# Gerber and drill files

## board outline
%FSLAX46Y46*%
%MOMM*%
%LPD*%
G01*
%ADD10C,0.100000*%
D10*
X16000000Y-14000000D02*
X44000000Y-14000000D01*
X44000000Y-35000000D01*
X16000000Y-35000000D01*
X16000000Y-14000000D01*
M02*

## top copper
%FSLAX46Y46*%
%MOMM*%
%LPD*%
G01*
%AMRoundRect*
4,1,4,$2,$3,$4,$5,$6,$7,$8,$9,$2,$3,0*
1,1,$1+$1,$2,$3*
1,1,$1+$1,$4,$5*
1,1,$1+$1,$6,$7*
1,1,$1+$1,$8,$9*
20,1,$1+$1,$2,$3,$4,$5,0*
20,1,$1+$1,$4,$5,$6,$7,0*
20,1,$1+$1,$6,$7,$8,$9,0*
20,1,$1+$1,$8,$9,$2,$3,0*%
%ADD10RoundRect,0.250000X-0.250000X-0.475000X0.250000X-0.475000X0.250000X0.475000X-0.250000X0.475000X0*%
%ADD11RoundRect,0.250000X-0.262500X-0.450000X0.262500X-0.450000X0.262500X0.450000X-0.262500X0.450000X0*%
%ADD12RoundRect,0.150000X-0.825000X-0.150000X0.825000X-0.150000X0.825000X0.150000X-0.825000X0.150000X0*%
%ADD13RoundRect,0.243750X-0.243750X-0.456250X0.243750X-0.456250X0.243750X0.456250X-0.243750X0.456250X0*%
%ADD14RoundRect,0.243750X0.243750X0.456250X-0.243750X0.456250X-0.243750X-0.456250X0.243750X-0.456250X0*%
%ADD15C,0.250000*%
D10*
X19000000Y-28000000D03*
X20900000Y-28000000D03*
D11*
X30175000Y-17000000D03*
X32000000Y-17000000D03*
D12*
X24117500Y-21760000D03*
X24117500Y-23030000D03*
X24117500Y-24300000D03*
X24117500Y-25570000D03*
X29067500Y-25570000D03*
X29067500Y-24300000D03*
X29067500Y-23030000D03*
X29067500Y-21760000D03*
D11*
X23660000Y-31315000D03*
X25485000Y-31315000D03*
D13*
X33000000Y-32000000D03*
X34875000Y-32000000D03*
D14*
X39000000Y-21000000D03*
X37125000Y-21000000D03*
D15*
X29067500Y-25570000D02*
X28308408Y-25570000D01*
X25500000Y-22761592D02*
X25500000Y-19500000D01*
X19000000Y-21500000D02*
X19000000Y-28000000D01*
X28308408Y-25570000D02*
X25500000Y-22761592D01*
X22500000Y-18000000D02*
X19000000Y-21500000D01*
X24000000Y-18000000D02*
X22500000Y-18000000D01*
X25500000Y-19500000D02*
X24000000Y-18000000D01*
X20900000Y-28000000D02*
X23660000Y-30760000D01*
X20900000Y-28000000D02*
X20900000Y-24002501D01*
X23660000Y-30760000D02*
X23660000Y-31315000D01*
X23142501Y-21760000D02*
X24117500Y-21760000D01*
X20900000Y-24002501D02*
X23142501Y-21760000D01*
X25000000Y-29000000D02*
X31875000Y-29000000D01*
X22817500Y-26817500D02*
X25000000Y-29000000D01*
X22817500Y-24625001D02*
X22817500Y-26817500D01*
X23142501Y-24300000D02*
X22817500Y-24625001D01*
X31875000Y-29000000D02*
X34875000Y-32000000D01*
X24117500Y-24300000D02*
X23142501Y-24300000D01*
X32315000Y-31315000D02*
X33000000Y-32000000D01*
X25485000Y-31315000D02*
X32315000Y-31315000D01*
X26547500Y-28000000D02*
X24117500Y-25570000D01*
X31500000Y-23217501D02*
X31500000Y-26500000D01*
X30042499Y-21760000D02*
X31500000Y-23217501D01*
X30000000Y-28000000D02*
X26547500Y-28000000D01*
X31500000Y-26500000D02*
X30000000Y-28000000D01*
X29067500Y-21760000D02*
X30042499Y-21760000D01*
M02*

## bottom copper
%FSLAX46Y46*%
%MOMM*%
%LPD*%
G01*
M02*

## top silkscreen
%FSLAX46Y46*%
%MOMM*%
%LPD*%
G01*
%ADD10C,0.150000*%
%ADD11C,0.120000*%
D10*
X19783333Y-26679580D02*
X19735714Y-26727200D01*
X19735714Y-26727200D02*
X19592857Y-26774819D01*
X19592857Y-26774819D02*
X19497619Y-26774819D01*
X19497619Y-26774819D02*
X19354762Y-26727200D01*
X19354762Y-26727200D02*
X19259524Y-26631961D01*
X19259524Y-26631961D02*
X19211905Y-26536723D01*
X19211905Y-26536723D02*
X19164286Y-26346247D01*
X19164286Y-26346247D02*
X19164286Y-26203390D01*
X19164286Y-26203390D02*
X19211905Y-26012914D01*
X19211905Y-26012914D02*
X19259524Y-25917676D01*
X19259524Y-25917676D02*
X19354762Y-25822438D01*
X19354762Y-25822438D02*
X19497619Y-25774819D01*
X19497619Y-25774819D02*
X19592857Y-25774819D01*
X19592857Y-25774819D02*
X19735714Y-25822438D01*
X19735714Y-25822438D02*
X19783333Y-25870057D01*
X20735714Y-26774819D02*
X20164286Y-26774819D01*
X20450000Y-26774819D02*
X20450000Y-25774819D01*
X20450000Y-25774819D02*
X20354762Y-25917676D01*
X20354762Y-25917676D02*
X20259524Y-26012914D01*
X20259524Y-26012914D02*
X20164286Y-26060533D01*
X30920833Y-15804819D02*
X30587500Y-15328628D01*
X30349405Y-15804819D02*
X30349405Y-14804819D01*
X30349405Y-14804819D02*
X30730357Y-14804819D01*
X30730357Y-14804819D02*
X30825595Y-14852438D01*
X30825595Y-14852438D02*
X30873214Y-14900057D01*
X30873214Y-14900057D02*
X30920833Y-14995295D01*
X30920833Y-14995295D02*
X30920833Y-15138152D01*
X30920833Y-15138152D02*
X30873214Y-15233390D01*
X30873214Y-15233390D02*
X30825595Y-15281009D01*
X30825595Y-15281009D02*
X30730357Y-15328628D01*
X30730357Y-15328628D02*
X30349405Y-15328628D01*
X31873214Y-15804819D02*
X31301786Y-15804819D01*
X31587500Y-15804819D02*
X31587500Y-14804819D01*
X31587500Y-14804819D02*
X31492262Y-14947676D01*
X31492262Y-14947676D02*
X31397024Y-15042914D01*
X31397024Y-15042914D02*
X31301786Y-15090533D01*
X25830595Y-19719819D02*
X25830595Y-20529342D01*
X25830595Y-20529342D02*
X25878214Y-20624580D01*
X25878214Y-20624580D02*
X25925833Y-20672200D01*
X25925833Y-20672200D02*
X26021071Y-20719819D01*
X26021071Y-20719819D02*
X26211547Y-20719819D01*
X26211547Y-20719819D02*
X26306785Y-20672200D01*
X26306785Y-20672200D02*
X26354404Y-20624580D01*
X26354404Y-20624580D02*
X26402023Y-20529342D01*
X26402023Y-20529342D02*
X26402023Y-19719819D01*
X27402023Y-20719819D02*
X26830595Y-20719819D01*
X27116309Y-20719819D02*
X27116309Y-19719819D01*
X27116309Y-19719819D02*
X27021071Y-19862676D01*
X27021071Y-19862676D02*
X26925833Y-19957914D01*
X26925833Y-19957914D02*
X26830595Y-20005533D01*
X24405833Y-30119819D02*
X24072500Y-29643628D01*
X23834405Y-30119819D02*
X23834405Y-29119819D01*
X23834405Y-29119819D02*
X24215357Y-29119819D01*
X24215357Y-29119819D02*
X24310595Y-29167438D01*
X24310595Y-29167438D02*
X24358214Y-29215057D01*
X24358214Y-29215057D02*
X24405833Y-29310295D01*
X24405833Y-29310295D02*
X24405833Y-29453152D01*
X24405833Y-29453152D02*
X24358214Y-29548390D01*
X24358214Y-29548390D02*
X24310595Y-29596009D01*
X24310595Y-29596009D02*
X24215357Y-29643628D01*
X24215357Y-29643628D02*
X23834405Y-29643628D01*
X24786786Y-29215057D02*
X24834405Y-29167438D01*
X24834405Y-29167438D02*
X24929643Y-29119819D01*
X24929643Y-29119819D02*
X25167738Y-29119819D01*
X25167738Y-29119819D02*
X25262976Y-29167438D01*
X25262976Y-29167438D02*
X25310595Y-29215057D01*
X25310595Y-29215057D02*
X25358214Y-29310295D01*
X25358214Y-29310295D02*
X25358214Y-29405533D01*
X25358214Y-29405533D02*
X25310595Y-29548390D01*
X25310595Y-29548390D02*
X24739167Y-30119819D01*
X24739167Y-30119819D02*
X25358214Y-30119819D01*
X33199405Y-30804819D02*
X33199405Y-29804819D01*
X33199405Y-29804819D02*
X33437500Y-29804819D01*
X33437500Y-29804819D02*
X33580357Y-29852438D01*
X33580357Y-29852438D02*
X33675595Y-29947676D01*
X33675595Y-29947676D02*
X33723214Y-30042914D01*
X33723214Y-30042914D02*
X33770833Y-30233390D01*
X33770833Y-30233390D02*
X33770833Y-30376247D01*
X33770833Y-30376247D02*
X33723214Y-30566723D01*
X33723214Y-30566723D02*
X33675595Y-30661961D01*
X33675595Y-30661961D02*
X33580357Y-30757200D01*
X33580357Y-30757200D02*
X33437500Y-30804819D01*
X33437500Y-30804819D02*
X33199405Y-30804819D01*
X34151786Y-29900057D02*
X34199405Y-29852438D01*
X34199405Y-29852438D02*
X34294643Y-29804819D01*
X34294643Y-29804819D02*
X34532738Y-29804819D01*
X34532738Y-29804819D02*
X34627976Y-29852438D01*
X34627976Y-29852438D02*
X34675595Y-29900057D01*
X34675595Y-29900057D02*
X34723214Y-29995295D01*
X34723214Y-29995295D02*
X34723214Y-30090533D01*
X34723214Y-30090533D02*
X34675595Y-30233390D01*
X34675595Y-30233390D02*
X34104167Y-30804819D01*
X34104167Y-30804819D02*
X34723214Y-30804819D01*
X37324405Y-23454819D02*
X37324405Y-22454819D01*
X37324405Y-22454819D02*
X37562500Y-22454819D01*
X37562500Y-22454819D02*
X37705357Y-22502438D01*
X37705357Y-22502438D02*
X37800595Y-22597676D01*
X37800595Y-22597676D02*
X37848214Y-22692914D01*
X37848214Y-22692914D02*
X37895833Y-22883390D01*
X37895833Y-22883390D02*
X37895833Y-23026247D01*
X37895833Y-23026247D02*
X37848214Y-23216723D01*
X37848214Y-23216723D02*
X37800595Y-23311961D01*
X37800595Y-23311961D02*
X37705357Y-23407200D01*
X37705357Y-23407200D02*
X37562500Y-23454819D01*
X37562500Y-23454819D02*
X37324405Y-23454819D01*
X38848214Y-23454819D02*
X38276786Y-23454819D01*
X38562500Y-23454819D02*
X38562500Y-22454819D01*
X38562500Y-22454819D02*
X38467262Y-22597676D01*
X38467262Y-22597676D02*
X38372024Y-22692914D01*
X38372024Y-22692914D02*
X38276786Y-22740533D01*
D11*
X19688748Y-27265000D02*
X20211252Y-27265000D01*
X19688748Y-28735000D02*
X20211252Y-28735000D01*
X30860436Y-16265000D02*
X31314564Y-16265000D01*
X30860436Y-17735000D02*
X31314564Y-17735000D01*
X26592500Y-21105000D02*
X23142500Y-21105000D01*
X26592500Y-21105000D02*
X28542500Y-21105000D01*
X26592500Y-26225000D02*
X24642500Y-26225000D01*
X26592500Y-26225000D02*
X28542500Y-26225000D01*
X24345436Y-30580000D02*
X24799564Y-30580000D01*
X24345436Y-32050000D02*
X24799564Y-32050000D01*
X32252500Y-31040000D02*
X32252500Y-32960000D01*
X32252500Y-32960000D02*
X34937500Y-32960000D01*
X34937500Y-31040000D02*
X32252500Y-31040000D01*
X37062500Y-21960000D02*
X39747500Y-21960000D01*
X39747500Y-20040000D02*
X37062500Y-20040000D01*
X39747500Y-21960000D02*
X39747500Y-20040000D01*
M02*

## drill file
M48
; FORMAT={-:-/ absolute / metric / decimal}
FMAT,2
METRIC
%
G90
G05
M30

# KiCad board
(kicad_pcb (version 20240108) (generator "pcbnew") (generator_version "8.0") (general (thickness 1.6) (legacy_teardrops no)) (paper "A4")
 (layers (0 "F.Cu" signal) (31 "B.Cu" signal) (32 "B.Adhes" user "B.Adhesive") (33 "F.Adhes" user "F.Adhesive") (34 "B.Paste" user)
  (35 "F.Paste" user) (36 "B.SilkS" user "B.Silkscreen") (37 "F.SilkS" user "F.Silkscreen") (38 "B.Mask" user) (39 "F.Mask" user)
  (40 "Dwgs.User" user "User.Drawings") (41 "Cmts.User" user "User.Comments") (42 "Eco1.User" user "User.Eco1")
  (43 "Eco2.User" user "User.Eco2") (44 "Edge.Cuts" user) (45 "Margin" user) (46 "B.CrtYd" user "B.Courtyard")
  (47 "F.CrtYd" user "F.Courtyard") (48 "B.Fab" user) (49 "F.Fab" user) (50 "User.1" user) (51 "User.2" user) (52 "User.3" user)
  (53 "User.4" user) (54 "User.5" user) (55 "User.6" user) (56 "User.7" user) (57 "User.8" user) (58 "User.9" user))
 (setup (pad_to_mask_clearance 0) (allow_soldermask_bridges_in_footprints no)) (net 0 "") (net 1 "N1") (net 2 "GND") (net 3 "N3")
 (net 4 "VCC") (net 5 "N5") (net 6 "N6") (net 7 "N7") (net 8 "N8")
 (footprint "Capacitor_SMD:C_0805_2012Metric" (layer "F.Cu") (at 19.95 28)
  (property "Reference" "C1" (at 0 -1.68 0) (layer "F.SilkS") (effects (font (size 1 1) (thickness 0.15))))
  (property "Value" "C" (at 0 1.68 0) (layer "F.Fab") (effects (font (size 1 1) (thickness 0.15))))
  (fp_line (start -0.261252 -0.735) (end 0.261252 -0.735) (stroke (width 0.12) (type solid)) (layer "F.SilkS"))
  (fp_line (start -0.261252 0.735) (end 0.261252 0.735) (stroke (width 0.12) (type solid)) (layer "F.SilkS"))
  (pad "1" smd roundrect (at -0.95 0) (size 1 1.45) (layers "F.Cu" "F.Paste" "F.Mask") (roundrect_rratio 0.25) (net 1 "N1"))
  (pad "2" smd roundrect (at 0.95 0) (size 1 1.45) (layers "F.Cu" "F.Paste" "F.Mask") (roundrect_rratio 0.25) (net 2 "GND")))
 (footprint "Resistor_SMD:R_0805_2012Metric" (layer "F.Cu") (at 31.0875 17)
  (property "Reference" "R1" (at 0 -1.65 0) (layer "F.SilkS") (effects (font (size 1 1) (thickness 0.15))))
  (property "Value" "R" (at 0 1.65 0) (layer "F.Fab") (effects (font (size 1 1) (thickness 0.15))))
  (fp_line (start -0.227064 -0.735) (end 0.227064 -0.735) (stroke (width 0.12) (type solid)) (layer "F.SilkS"))
  (fp_line (start -0.227064 0.735) (end 0.227064 0.735) (stroke (width 0.12) (type solid)) (layer "F.SilkS"))
  (pad "1" smd roundrect (at -0.9125 0) (size 1.025 1.4) (layers "F.Cu" "F.Paste" "F.Mask") (roundrect_rratio 0.243902) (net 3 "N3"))
  (pad "2" smd roundrect (at 0.9125 0) (size 1.025 1.4) (layers "F.Cu" "F.Paste" "F.Mask") (roundrect_rratio 0.243902) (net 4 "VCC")))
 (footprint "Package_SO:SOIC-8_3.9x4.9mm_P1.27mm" (layer "F.Cu") (at 26.5925 23.665)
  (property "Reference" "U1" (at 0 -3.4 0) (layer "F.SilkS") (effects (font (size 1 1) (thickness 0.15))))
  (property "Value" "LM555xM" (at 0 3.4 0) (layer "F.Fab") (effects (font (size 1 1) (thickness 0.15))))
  (fp_line (start 0 -2.56) (end -3.45 -2.56) (stroke (width 0.12) (type solid)) (layer "F.SilkS"))
  (fp_line (start 0 -2.56) (end 1.95 -2.56) (stroke (width 0.12) (type solid)) (layer "F.SilkS"))
  (fp_line (start 0 2.56) (end -1.95 2.56) (stroke (width 0.12) (type solid)) (layer "F.SilkS"))
  (fp_line (start 0 2.56) (end 1.95 2.56) (stroke (width 0.12) (type solid)) (layer "F.SilkS"))
  (pad "1" smd roundrect (at -2.475 -1.905) (size 1.95 0.6) (layers "F.Cu" "F.Paste" "F.Mask") (roundrect_rratio 0.25) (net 2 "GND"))
  (pad "2" smd roundrect (at -2.475 -0.635) (size 1.95 0.6) (layers "F.Cu" "F.Paste" "F.Mask") (roundrect_rratio 0.25) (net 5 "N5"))
  (pad "3" smd roundrect (at -2.475 0.635) (size 1.95 0.6) (layers "F.Cu" "F.Paste" "F.Mask") (roundrect_rratio 0.25) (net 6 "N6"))
  (pad "4" smd roundrect (at -2.475 1.905) (size 1.95 0.6) (layers "F.Cu" "F.Paste" "F.Mask") (roundrect_rratio 0.25) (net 4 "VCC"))
  (pad "5" smd roundrect (at 2.475 1.905) (size 1.95 0.6) (layers "F.Cu" "F.Paste" "F.Mask") (roundrect_rratio 0.25) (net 1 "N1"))
  (pad "6" smd roundrect (at 2.475 0.635) (size 1.95 0.6) (layers "F.Cu" "F.Paste" "F.Mask") (roundrect_rratio 0.25) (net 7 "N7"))
  (pad "7" smd roundrect (at 2.475 -0.635) (size 1.95 0.6) (layers "F.Cu" "F.Paste" "F.Mask") (roundrect_rratio 0.25) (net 7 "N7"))
  (pad "8" smd roundrect (at 2.475 -1.905) (size 1.95 0.6) (layers "F.Cu" "F.Paste" "F.Mask") (roundrect_rratio 0.25) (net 4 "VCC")))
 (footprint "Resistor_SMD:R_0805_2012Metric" (layer "F.Cu") (at 24.5725 31.315)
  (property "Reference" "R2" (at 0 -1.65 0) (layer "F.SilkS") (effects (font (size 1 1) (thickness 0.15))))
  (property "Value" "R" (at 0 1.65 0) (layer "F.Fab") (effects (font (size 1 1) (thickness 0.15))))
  (fp_line (start -0.227064 -0.735) (end 0.227064 -0.735) (stroke (width 0.12) (type solid)) (layer "F.SilkS"))
  (fp_line (start -0.227064 0.735) (end 0.227064 0.735) (stroke (width 0.12) (type solid)) (layer "F.SilkS"))
  (pad "1" smd roundrect (at -0.9125 0) (size 1.025 1.4) (layers "F.Cu" "F.Paste" "F.Mask") (roundrect_rratio 0.243902) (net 2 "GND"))
  (pad "2" smd roundrect (at 0.9125 0) (size 1.025 1.4) (layers "F.Cu" "F.Paste" "F.Mask") (roundrect_rratio 0.243902) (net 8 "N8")))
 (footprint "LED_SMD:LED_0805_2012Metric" (layer "F.Cu") (at 33.9375 32)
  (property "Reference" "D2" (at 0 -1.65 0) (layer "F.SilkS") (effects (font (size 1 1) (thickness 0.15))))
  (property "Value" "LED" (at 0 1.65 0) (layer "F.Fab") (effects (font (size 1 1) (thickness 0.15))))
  (fp_line (start -1.685 -0.96) (end -1.685 0.96) (stroke (width 0.12) (type solid)) (layer "F.SilkS"))
  (fp_line (start -1.685 0.96) (end 1 0.96) (stroke (width 0.12) (type solid)) (layer "F.SilkS"))
  (fp_line (start 1 -0.96) (end -1.685 -0.96) (stroke (width 0.12) (type solid)) (layer "F.SilkS"))
  (pad "1" smd roundrect (at -0.9375 0) (size 0.975 1.4) (layers "F.Cu" "F.Paste" "F.Mask") (roundrect_rratio 0.25) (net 8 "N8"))
  (pad "2" smd roundrect (at 0.9375 0) (size 0.975 1.4) (layers "F.Cu" "F.Paste" "F.Mask") (roundrect_rratio 0.25) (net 6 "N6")))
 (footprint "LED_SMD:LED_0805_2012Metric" (layer "F.Cu") (at 38.0625 21 180)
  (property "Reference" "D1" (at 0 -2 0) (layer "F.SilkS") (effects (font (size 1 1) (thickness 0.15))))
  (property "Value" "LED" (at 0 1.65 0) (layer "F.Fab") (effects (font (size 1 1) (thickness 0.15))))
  (fp_line (start 1 -0.96) (end -1.685 -0.96) (stroke (width 0.12) (type solid)) (layer "F.SilkS"))
  (fp_line (start -1.685 0.96) (end 1 0.96) (stroke (width 0.12) (type solid)) (layer "F.SilkS"))
  (fp_line (start -1.685 -0.96) (end -1.685 0.96) (stroke (width 0.12) (type solid)) (layer "F.SilkS"))
  (pad "1" smd roundrect (at -0.9375 0 180) (size 0.975 1.4) (layers "F.Cu" "F.Paste" "F.Mask") (roundrect_rratio 0.25) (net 6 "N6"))
  (pad "2" smd roundrect (at 0.9375 0 180) (size 0.975 1.4) (layers "F.Cu" "F.Paste" "F.Mask") (roundrect_rratio 0.25) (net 3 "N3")))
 (gr_rect (start 16 14) (end 44 35) (stroke (width 0.1) (type default)) (fill none) (layer "Edge.Cuts"))
 (segment (start 29.0675 25.57) (end 28.308408 25.57) (width 0.25) (layer "F.Cu") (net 1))
 (segment (start 25.5 22.761592) (end 25.5 19.5) (width 0.25) (layer "F.Cu") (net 1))
 (segment (start 19 21.5) (end 19 28) (width 0.25) (layer "F.Cu") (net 1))
 (segment (start 28.308408 25.57) (end 25.5 22.761592) (width 0.25) (layer "F.Cu") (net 1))
 (segment (start 22.5 18) (end 19 21.5) (width 0.25) (layer "F.Cu") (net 1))
 (segment (start 24 18) (end 22.5 18) (width 0.25) (layer "F.Cu") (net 1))
 (segment (start 25.5 19.5) (end 24 18) (width 0.25) (layer "F.Cu") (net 1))
 (segment (start 20.9 28) (end 23.66 30.76) (width 0.25) (layer "F.Cu") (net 2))
 (segment (start 20.9 28) (end 20.9 24.002501) (width 0.25) (layer "F.Cu") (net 2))
 (segment (start 23.66 30.76) (end 23.66 31.315) (width 0.25) (layer "F.Cu") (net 2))
 (segment (start 23.142501 21.76) (end 24.1175 21.76) (width 0.25) (layer "F.Cu") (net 2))
 (segment (start 20.9 24.002501) (end 23.142501 21.76) (width 0.25) (layer "F.Cu") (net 2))
 (segment (start 25 29) (end 31.875 29) (width 0.25) (layer "F.Cu") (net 6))
 (segment (start 22.8175 26.8175) (end 25 29) (width 0.25) (layer "F.Cu") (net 6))
 (segment (start 22.8175 24.625001) (end 22.8175 26.8175) (width 0.25) (layer "F.Cu") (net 6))
 (segment (start 23.142501 24.3) (end 22.8175 24.625001) (width 0.25) (layer "F.Cu") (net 6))
 (segment (start 31.875 29) (end 34.875 32) (width 0.25) (layer "F.Cu") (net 6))
 (segment (start 24.1175 24.3) (end 23.142501 24.3) (width 0.25) (layer "F.Cu") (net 6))
 (segment (start 32.315 31.315) (end 33 32) (width 0.25) (layer "F.Cu") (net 8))
 (segment (start 25.485 31.315) (end 32.315 31.315) (width 0.25) (layer "F.Cu") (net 8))
 (segment (start 26.5475 28) (end 24.1175 25.57) (width 0.25) (layer "F.Cu") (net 4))
 (segment (start 31.5 23.217501) (end 31.5 26.5) (width 0.25) (layer "F.Cu") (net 4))
 (segment (start 30.042499 21.76) (end 31.5 23.217501) (width 0.25) (layer "F.Cu") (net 4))
 (segment (start 30 28) (end 26.5475 28) (width 0.25) (layer "F.Cu") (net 4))
 (segment (start 31.5 26.5) (end 30 28) (width 0.25) (layer "F.Cu") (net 4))
 (segment (start 29.0675 21.76) (end 30.042499 21.76) (width 0.25) (layer "F.Cu") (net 4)))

